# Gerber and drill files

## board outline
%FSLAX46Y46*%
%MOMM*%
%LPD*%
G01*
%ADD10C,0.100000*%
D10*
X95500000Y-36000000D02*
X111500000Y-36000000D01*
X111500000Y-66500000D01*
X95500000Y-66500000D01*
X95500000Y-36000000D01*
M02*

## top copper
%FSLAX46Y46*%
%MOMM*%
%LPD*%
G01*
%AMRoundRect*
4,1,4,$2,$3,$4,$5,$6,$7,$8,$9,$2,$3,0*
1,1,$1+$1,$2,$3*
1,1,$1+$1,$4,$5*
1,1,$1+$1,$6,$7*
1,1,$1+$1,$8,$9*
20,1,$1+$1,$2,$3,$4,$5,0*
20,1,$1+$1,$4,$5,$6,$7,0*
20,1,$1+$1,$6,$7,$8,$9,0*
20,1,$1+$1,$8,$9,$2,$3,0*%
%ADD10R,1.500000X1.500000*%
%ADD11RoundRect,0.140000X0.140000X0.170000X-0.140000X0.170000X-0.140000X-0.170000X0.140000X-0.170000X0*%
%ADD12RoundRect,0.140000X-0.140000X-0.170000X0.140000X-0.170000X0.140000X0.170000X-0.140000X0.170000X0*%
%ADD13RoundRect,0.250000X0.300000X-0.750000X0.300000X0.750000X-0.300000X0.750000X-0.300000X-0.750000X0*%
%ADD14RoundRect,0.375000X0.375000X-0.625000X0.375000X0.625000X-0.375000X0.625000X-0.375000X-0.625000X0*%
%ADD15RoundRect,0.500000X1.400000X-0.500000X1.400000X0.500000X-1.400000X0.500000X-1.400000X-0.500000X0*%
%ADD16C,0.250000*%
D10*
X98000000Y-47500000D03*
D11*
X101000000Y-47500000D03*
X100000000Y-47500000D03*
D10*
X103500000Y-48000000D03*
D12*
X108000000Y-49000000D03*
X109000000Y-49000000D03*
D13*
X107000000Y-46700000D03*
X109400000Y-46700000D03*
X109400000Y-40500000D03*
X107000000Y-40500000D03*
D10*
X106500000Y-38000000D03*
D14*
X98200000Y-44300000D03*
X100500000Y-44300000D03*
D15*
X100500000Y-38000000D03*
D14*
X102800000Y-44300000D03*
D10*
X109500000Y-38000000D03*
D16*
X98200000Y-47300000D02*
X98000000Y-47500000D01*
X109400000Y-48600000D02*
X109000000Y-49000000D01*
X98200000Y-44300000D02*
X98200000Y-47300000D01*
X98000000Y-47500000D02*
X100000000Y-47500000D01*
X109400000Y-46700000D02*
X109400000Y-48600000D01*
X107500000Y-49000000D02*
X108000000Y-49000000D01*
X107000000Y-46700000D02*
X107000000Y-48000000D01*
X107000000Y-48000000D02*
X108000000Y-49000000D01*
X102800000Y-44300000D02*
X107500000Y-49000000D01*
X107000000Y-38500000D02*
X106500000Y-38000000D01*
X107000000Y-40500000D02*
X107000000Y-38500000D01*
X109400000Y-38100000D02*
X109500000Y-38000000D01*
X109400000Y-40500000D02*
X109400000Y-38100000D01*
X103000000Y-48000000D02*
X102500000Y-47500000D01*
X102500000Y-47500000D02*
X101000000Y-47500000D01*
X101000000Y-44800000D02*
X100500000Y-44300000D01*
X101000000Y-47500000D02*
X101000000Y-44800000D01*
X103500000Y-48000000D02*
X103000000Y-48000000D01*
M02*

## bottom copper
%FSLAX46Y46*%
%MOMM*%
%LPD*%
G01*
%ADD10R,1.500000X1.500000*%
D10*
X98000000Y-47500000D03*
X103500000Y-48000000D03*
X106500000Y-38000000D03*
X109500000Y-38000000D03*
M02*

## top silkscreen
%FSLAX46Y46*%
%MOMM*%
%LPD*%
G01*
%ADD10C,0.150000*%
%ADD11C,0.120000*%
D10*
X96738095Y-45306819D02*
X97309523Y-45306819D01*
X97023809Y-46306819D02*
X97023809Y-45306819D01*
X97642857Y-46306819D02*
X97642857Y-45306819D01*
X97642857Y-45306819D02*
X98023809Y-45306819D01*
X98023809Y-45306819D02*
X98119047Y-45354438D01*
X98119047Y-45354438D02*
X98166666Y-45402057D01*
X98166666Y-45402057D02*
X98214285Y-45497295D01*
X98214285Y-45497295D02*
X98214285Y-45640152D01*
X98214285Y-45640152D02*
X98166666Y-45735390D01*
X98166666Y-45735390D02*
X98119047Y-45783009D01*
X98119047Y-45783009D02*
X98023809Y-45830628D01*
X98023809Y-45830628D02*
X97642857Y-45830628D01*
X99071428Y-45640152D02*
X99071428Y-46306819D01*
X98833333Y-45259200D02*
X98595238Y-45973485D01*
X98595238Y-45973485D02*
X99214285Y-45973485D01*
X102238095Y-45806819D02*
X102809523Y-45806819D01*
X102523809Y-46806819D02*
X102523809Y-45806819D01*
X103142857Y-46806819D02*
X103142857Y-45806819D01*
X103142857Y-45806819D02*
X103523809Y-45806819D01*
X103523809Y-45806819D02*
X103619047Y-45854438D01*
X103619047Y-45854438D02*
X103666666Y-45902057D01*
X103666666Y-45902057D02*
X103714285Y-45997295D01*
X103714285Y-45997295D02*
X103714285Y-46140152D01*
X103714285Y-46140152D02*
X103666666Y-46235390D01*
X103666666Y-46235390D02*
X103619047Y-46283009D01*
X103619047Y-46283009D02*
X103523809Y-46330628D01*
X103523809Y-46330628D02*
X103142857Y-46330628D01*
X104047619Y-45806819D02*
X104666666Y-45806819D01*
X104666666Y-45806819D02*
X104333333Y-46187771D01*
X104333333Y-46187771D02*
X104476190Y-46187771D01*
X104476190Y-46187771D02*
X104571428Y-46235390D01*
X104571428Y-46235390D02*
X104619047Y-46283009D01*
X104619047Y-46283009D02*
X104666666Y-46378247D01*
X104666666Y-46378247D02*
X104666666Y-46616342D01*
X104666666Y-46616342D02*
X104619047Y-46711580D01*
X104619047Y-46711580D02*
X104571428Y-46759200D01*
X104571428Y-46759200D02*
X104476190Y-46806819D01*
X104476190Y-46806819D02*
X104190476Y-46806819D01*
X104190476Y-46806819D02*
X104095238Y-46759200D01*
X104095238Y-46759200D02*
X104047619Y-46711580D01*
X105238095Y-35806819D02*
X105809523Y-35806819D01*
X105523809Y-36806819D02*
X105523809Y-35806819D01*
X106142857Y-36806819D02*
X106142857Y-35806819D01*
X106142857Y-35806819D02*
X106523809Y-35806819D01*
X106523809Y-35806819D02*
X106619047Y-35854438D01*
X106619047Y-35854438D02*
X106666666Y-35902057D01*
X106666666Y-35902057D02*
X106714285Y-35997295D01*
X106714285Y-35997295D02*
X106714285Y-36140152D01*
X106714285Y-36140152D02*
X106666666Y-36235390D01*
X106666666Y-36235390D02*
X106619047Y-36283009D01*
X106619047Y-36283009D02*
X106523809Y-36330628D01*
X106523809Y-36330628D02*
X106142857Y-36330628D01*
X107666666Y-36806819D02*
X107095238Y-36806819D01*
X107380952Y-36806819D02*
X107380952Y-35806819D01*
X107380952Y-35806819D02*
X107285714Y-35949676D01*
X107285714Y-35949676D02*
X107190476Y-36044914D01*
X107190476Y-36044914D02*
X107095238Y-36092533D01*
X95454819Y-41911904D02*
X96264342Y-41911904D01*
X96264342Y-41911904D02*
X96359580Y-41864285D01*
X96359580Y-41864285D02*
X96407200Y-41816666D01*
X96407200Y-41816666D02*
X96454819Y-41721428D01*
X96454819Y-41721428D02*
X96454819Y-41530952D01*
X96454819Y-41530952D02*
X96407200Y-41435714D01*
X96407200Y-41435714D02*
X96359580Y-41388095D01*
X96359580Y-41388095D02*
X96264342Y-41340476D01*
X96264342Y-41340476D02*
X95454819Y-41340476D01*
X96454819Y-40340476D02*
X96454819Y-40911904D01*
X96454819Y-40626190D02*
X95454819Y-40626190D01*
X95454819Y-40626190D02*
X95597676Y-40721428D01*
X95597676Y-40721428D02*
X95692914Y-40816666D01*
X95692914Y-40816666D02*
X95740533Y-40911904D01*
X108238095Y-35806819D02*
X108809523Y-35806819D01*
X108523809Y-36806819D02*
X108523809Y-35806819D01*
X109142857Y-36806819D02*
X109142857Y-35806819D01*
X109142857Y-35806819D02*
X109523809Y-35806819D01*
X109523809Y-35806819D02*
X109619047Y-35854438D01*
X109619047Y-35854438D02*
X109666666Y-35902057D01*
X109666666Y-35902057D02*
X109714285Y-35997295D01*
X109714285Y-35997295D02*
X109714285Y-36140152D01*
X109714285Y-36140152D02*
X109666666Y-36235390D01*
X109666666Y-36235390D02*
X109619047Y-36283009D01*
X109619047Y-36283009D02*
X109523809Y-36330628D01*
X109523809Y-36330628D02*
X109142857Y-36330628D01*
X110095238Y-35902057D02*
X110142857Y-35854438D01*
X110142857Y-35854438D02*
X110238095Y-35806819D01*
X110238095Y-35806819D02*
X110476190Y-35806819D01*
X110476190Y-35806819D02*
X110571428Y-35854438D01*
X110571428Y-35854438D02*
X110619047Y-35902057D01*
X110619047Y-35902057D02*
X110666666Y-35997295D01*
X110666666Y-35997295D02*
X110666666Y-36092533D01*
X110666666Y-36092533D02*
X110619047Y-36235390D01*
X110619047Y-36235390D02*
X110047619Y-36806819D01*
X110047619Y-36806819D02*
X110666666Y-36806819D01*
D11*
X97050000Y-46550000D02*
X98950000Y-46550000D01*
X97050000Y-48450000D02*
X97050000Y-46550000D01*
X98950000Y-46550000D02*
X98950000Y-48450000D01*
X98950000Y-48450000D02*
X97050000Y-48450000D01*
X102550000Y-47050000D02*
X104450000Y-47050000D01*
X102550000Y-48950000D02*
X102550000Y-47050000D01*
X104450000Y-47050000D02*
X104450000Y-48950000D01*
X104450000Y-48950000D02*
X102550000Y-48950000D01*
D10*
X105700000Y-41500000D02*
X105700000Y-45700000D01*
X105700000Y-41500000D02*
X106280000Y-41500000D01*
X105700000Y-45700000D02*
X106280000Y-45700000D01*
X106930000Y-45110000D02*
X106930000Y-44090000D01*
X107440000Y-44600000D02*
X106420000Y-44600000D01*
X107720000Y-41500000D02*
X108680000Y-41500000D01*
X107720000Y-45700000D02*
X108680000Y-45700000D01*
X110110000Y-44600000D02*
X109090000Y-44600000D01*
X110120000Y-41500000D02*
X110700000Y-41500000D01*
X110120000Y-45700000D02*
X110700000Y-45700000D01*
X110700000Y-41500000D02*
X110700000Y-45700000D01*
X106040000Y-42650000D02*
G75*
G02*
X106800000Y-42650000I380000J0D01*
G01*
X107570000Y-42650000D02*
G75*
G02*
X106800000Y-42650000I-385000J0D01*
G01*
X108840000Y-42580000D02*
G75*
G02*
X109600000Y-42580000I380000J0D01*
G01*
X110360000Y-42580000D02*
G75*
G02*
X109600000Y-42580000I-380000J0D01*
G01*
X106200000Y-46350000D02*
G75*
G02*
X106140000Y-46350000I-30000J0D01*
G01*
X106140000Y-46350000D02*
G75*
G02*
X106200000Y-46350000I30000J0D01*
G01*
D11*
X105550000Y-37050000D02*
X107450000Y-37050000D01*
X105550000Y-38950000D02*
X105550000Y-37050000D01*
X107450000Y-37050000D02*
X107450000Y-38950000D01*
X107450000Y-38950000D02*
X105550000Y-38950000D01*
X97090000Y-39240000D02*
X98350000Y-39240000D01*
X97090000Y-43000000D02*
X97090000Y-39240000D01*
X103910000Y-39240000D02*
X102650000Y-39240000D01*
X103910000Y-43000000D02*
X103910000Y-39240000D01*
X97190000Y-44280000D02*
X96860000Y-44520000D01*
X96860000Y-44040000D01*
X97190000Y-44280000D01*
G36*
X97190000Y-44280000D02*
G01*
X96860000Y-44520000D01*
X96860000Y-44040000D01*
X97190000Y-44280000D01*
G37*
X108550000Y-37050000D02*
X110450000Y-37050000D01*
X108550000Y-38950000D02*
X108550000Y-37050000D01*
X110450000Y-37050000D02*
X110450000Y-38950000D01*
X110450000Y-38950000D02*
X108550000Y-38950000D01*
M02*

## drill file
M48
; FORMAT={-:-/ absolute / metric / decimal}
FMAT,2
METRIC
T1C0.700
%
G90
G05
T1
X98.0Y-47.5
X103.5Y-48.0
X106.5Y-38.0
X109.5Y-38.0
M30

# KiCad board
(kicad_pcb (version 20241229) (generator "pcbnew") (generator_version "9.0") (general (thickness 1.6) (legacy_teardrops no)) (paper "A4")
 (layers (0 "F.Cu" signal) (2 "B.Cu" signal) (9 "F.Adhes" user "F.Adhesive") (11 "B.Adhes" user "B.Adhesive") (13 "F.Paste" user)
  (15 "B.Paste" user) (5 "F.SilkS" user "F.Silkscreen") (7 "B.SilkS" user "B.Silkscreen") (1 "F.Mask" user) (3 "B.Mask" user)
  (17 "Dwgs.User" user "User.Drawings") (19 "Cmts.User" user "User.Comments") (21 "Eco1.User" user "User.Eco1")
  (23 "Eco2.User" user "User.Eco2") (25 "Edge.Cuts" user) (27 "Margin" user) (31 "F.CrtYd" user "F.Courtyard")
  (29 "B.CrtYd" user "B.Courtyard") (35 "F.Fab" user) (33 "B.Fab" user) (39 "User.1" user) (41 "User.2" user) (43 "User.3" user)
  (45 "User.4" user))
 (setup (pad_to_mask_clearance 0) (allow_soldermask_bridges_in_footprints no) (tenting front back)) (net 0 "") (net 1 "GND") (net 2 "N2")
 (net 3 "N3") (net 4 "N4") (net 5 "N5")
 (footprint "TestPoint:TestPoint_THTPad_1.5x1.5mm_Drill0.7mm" (layer "F.Cu") (at 98 47.5)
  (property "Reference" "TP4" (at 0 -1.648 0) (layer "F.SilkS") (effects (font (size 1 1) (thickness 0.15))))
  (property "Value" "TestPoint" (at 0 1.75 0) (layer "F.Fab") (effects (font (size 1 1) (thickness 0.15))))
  (fp_line (start -0.95 -0.95) (end 0.95 -0.95) (stroke (width 0.12) (type solid)) (layer "F.SilkS"))
  (fp_line (start -0.95 0.95) (end -0.95 -0.95) (stroke (width 0.12) (type solid)) (layer "F.SilkS"))
  (fp_line (start 0.95 -0.95) (end 0.95 0.95) (stroke (width 0.12) (type solid)) (layer "F.SilkS"))
  (fp_line (start 0.95 0.95) (end -0.95 0.95) (stroke (width 0.12) (type solid)) (layer "F.SilkS"))
  (pad "1" thru_hole rect (at 0 0) (size 1.5 1.5) (drill 0.7) (layers "*.Cu" "*.Mask") (remove_unused_layers no) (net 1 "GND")))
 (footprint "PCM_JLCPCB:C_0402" (layer "F.Cu") (at 100.5 47.5 180)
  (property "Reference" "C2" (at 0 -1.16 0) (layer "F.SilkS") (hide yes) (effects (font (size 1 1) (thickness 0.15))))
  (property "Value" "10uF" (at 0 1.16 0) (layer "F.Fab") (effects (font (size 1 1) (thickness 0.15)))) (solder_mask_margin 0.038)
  (pad "1" smd roundrect (at -0.5 0 180) (size 0.56 0.62) (layers "F.Cu" "F.Mask" "F.Paste") (roundrect_rratio 0.25) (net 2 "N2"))
  (pad "2" smd roundrect (at 0.5 0 180) (size 0.56 0.62) (layers "F.Cu" "F.Mask" "F.Paste") (roundrect_rratio 0.25) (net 1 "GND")))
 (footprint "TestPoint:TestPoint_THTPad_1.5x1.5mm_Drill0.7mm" (layer "F.Cu") (at 103.5 48)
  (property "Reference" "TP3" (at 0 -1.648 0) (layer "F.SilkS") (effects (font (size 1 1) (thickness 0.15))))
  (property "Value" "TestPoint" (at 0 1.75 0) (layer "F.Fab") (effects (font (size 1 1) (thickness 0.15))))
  (fp_line (start -0.95 -0.95) (end 0.95 -0.95) (stroke (width 0.12) (type solid)) (layer "F.SilkS"))
  (fp_line (start -0.95 0.95) (end -0.95 -0.95) (stroke (width 0.12) (type solid)) (layer "F.SilkS"))
  (fp_line (start 0.95 -0.95) (end 0.95 0.95) (stroke (width 0.12) (type solid)) (layer "F.SilkS"))
  (fp_line (start 0.95 0.95) (end -0.95 0.95) (stroke (width 0.12) (type solid)) (layer "F.SilkS"))
  (pad "1" thru_hole rect (at 0 0) (size 1.5 1.5) (drill 0.7) (layers "*.Cu" "*.Mask") (remove_unused_layers no) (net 2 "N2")))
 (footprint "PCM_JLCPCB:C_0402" (layer "F.Cu") (at 108.5 49)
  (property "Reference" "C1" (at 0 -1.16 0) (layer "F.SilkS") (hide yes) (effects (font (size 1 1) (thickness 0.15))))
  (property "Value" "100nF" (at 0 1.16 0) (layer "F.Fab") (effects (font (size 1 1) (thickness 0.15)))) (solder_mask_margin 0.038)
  (pad "1" smd roundrect (at -0.5 0) (size 0.56 0.62) (layers "F.Cu" "F.Mask" "F.Paste") (roundrect_rratio 0.25) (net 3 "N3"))
  (pad "2" smd roundrect (at 0.5 0) (size 0.56 0.62) (layers "F.Cu" "F.Mask" "F.Paste") (roundrect_rratio 0.25) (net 1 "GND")))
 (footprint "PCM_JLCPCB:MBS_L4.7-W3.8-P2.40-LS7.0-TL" (layer "F.Cu") (at 108.2 43.6 90)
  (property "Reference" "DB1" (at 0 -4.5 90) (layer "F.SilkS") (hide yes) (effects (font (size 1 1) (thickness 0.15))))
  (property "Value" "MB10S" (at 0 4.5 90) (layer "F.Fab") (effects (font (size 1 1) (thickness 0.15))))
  (fp_line (start 2.1 -2.5) (end -2.1 -2.5) (stroke (width 0.15) (type solid)) (layer "F.SilkS"))
  (fp_line (start 2.1 -2.5) (end 2.1 -1.92) (stroke (width 0.15) (type solid)) (layer "F.SilkS"))
  (fp_line (start -2.1 -2.5) (end -2.1 -1.92) (stroke (width 0.15) (type solid)) (layer "F.SilkS"))
  (fp_line (start -1.51 -1.27) (end -0.49 -1.27) (stroke (width 0.15) (type solid)) (layer "F.SilkS"))
  (fp_line (start -1 -0.76) (end -1 -1.78) (stroke (width 0.15) (type solid)) (layer "F.SilkS"))
  (fp_line (start 2.1 -0.48) (end 2.1 0.48) (stroke (width 0.15) (type solid)) (layer "F.SilkS"))
  (fp_line (start -2.1 -0.48) (end -2.1 0.48) (stroke (width 0.15) (type solid)) (layer "F.SilkS"))
  (fp_line (start -1 1.91) (end -1 0.89) (stroke (width 0.15) (type solid)) (layer "F.SilkS"))
  (fp_line (start 2.1 1.92) (end 2.1 2.5) (stroke (width 0.15) (type solid)) (layer "F.SilkS"))
  (fp_line (start -2.1 1.92) (end -2.1 2.5) (stroke (width 0.15) (type solid)) (layer "F.SilkS"))
  (fp_line (start 2.1 2.5) (end -2.1 2.5) (stroke (width 0.15) (type solid)) (layer "F.SilkS"))
  (fp_arc (start 0.95 -2.16) (mid 1.33 -1.78) (end 0.95 -1.4) (stroke (width 0.15) (type solid)) (layer "F.SilkS"))
  (fp_arc (start 0.95 -0.63) (mid 0.565 -1.015) (end 0.95 -1.4) (stroke (width 0.15) (type solid)) (layer "F.SilkS"))
  (fp_arc (start 1.02 0.64) (mid 1.4 1.02) (end 1.02 1.4) (stroke (width 0.15) (type solid)) (layer "F.SilkS"))
  (fp_arc (start 1.02 2.16) (mid 0.64 1.78) (end 1.02 1.4) (stroke (width 0.15) (type solid)) (layer "F.SilkS"))
  (fp_circle (center -2.75 -2.03) (end -2.72 -2.03) (stroke (width 0.15) (type solid)) (fill no) (layer "F.SilkS"))
  (pad "1" smd roundrect (at -3.1 -1.2 90) (size 2 1.1) (layers "F.Cu" "F.Mask" "F.Paste") (roundrect_rratio 0.2272727273) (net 3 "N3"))
  (pad "2" smd roundrect (at -3.1 1.2 90) (size 2 1.1) (layers "F.Cu" "F.Mask" "F.Paste") (roundrect_rratio 0.2272727273) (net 1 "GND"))
  (pad "3" smd roundrect (at 3.1 1.2 90) (size 2 1.1) (layers "F.Cu" "F.Mask" "F.Paste") (roundrect_rratio 0.2272727273) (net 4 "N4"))
  (pad "4" smd roundrect (at 3.1 -1.2 90) (size 2 1.1) (layers "F.Cu" "F.Mask" "F.Paste") (roundrect_rratio 0.2272727273) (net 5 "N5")))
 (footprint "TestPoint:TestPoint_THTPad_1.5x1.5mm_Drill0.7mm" (layer "F.Cu") (at 106.5 38)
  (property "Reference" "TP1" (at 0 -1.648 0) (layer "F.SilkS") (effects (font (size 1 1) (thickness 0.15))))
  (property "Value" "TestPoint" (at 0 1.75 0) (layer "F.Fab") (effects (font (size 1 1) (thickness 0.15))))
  (fp_line (start -0.95 -0.95) (end 0.95 -0.95) (stroke (width 0.12) (type solid)) (layer "F.SilkS"))
  (fp_line (start -0.95 0.95) (end -0.95 -0.95) (stroke (width 0.12) (type solid)) (layer "F.SilkS"))
  (fp_line (start 0.95 -0.95) (end 0.95 0.95) (stroke (width 0.12) (type solid)) (layer "F.SilkS"))
  (fp_line (start 0.95 0.95) (end -0.95 0.95) (stroke (width 0.12) (type solid)) (layer "F.SilkS"))
  (pad "1" thru_hole rect (at 0 0) (size 1.5 1.5) (drill 0.7) (layers "*.Cu" "*.Mask") (remove_unused_layers no) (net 5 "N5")))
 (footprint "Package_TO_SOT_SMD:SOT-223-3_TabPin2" (layer "F.Cu") (at 100.5 41.15 90)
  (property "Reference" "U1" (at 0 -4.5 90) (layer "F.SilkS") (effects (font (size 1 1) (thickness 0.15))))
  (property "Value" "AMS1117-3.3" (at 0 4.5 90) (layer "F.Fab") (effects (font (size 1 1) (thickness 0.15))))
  (fp_line (start 1.91 -3.41) (end 1.91 -2.15) (stroke (width 0.12) (type solid)) (layer "F.SilkS"))
  (fp_line (start -1.85 -3.41) (end 1.91 -3.41) (stroke (width 0.12) (type solid)) (layer "F.SilkS"))
  (fp_line (start 1.91 3.41) (end 1.91 2.15) (stroke (width 0.12) (type solid)) (layer "F.SilkS"))
  (fp_line (start -1.85 3.41) (end 1.91 3.41) (stroke (width 0.12) (type solid)) (layer "F.SilkS"))
  (fp_poly
   (pts (xy -3.13 -3.31) (xy -3.37 -3.64) (xy -2.89 -3.64) (xy -3.13 -3.31)) (stroke (width 0.12) (type solid)) (fill yes) (layer "F.SilkS"))
  (pad "1" smd roundrect (at -3.15 -2.3 90) (size 2 1.5) (layers "F.Cu" "F.Mask" "F.Paste") (roundrect_rratio 0.25) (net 1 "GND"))
  (pad "2" smd roundrect (at -3.15 0 90) (size 2 1.5) (layers "F.Cu" "F.Mask" "F.Paste") (roundrect_rratio 0.25) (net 2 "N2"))
  (pad "2" smd roundrect (at 3.15 0 90) (size 2 3.8) (layers "F.Cu" "F.Mask" "F.Paste") (roundrect_rratio 0.25) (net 2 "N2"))
  (pad "3" smd roundrect (at -3.15 2.3 90) (size 2 1.5) (layers "F.Cu" "F.Mask" "F.Paste") (roundrect_rratio 0.25) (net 3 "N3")))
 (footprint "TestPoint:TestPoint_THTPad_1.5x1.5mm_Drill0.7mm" (layer "F.Cu") (at 109.5 38)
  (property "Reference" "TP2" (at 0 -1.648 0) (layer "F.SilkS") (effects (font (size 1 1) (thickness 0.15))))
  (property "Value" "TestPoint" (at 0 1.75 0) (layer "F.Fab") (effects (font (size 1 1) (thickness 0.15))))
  (fp_line (start -0.95 -0.95) (end 0.95 -0.95) (stroke (width 0.12) (type solid)) (layer "F.SilkS"))
  (fp_line (start -0.95 0.95) (end -0.95 -0.95) (stroke (width 0.12) (type solid)) (layer "F.SilkS"))
  (fp_line (start 0.95 -0.95) (end 0.95 0.95) (stroke (width 0.12) (type solid)) (layer "F.SilkS"))
  (fp_line (start 0.95 0.95) (end -0.95 0.95) (stroke (width 0.12) (type solid)) (layer "F.SilkS"))
  (pad "1" thru_hole rect (at 0 0) (size 1.5 1.5) (drill 0.7) (layers "*.Cu" "*.Mask") (remove_unused_layers no) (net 4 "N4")))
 (gr_rect (start 95.5 36) (end 111.5 66.5) (stroke (width 0.1) (type default)) (fill no) (layer "Edge.Cuts"))
 (segment (start 98.2 47.3) (end 98 47.5) (width 0.25) (layer "F.Cu") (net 1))
 (segment (start 109.4 48.6) (end 109 49) (width 0.25) (layer "F.Cu") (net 1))
 (segment (start 98.2 44.3) (end 98.2 47.3) (width 0.25) (layer "F.Cu") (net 1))
 (segment (start 98 47.5) (end 100 47.5) (width 0.25) (layer "F.Cu") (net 1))
 (segment (start 109.4 46.7) (end 109.4 48.6) (width 0.25) (layer "F.Cu") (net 1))
 (segment (start 107.5 49) (end 108 49) (width 0.25) (layer "F.Cu") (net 3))
 (segment (start 107 46.7) (end 107 48) (width 0.25) (layer "F.Cu") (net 3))
 (segment (start 107 48) (end 108 49) (width 0.25) (layer "F.Cu") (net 3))
 (segment (start 102.8 44.3) (end 107.5 49) (width 0.25) (layer "F.Cu") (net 3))
 (segment (start 107 38.5) (end 106.5 38) (width 0.25) (layer "F.Cu") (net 5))
 (segment (start 107 40.5) (end 107 38.5) (width 0.25) (layer "F.Cu") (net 5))
 (segment (start 109.4 38.1) (end 109.5 38) (width 0.25) (layer "F.Cu") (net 4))
 (segment (start 109.4 40.5) (end 109.4 38.1) (width 0.25) (layer "F.Cu") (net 4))
 (segment (start 103 48) (end 102.5 47.5) (width 0.25) (layer "F.Cu") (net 2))
 (segment (start 102.5 47.5) (end 101 47.5) (width 0.25) (layer "F.Cu") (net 2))
 (segment (start 101 44.8) (end 100.5 44.3) (width 0.25) (layer "F.Cu") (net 2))
 (segment (start 101 47.5) (end 101 44.8) (width 0.25) (layer "F.Cu") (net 2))
 (segment (start 103.5 48) (end 103 48) (width 0.25) (layer "F.Cu") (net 2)))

